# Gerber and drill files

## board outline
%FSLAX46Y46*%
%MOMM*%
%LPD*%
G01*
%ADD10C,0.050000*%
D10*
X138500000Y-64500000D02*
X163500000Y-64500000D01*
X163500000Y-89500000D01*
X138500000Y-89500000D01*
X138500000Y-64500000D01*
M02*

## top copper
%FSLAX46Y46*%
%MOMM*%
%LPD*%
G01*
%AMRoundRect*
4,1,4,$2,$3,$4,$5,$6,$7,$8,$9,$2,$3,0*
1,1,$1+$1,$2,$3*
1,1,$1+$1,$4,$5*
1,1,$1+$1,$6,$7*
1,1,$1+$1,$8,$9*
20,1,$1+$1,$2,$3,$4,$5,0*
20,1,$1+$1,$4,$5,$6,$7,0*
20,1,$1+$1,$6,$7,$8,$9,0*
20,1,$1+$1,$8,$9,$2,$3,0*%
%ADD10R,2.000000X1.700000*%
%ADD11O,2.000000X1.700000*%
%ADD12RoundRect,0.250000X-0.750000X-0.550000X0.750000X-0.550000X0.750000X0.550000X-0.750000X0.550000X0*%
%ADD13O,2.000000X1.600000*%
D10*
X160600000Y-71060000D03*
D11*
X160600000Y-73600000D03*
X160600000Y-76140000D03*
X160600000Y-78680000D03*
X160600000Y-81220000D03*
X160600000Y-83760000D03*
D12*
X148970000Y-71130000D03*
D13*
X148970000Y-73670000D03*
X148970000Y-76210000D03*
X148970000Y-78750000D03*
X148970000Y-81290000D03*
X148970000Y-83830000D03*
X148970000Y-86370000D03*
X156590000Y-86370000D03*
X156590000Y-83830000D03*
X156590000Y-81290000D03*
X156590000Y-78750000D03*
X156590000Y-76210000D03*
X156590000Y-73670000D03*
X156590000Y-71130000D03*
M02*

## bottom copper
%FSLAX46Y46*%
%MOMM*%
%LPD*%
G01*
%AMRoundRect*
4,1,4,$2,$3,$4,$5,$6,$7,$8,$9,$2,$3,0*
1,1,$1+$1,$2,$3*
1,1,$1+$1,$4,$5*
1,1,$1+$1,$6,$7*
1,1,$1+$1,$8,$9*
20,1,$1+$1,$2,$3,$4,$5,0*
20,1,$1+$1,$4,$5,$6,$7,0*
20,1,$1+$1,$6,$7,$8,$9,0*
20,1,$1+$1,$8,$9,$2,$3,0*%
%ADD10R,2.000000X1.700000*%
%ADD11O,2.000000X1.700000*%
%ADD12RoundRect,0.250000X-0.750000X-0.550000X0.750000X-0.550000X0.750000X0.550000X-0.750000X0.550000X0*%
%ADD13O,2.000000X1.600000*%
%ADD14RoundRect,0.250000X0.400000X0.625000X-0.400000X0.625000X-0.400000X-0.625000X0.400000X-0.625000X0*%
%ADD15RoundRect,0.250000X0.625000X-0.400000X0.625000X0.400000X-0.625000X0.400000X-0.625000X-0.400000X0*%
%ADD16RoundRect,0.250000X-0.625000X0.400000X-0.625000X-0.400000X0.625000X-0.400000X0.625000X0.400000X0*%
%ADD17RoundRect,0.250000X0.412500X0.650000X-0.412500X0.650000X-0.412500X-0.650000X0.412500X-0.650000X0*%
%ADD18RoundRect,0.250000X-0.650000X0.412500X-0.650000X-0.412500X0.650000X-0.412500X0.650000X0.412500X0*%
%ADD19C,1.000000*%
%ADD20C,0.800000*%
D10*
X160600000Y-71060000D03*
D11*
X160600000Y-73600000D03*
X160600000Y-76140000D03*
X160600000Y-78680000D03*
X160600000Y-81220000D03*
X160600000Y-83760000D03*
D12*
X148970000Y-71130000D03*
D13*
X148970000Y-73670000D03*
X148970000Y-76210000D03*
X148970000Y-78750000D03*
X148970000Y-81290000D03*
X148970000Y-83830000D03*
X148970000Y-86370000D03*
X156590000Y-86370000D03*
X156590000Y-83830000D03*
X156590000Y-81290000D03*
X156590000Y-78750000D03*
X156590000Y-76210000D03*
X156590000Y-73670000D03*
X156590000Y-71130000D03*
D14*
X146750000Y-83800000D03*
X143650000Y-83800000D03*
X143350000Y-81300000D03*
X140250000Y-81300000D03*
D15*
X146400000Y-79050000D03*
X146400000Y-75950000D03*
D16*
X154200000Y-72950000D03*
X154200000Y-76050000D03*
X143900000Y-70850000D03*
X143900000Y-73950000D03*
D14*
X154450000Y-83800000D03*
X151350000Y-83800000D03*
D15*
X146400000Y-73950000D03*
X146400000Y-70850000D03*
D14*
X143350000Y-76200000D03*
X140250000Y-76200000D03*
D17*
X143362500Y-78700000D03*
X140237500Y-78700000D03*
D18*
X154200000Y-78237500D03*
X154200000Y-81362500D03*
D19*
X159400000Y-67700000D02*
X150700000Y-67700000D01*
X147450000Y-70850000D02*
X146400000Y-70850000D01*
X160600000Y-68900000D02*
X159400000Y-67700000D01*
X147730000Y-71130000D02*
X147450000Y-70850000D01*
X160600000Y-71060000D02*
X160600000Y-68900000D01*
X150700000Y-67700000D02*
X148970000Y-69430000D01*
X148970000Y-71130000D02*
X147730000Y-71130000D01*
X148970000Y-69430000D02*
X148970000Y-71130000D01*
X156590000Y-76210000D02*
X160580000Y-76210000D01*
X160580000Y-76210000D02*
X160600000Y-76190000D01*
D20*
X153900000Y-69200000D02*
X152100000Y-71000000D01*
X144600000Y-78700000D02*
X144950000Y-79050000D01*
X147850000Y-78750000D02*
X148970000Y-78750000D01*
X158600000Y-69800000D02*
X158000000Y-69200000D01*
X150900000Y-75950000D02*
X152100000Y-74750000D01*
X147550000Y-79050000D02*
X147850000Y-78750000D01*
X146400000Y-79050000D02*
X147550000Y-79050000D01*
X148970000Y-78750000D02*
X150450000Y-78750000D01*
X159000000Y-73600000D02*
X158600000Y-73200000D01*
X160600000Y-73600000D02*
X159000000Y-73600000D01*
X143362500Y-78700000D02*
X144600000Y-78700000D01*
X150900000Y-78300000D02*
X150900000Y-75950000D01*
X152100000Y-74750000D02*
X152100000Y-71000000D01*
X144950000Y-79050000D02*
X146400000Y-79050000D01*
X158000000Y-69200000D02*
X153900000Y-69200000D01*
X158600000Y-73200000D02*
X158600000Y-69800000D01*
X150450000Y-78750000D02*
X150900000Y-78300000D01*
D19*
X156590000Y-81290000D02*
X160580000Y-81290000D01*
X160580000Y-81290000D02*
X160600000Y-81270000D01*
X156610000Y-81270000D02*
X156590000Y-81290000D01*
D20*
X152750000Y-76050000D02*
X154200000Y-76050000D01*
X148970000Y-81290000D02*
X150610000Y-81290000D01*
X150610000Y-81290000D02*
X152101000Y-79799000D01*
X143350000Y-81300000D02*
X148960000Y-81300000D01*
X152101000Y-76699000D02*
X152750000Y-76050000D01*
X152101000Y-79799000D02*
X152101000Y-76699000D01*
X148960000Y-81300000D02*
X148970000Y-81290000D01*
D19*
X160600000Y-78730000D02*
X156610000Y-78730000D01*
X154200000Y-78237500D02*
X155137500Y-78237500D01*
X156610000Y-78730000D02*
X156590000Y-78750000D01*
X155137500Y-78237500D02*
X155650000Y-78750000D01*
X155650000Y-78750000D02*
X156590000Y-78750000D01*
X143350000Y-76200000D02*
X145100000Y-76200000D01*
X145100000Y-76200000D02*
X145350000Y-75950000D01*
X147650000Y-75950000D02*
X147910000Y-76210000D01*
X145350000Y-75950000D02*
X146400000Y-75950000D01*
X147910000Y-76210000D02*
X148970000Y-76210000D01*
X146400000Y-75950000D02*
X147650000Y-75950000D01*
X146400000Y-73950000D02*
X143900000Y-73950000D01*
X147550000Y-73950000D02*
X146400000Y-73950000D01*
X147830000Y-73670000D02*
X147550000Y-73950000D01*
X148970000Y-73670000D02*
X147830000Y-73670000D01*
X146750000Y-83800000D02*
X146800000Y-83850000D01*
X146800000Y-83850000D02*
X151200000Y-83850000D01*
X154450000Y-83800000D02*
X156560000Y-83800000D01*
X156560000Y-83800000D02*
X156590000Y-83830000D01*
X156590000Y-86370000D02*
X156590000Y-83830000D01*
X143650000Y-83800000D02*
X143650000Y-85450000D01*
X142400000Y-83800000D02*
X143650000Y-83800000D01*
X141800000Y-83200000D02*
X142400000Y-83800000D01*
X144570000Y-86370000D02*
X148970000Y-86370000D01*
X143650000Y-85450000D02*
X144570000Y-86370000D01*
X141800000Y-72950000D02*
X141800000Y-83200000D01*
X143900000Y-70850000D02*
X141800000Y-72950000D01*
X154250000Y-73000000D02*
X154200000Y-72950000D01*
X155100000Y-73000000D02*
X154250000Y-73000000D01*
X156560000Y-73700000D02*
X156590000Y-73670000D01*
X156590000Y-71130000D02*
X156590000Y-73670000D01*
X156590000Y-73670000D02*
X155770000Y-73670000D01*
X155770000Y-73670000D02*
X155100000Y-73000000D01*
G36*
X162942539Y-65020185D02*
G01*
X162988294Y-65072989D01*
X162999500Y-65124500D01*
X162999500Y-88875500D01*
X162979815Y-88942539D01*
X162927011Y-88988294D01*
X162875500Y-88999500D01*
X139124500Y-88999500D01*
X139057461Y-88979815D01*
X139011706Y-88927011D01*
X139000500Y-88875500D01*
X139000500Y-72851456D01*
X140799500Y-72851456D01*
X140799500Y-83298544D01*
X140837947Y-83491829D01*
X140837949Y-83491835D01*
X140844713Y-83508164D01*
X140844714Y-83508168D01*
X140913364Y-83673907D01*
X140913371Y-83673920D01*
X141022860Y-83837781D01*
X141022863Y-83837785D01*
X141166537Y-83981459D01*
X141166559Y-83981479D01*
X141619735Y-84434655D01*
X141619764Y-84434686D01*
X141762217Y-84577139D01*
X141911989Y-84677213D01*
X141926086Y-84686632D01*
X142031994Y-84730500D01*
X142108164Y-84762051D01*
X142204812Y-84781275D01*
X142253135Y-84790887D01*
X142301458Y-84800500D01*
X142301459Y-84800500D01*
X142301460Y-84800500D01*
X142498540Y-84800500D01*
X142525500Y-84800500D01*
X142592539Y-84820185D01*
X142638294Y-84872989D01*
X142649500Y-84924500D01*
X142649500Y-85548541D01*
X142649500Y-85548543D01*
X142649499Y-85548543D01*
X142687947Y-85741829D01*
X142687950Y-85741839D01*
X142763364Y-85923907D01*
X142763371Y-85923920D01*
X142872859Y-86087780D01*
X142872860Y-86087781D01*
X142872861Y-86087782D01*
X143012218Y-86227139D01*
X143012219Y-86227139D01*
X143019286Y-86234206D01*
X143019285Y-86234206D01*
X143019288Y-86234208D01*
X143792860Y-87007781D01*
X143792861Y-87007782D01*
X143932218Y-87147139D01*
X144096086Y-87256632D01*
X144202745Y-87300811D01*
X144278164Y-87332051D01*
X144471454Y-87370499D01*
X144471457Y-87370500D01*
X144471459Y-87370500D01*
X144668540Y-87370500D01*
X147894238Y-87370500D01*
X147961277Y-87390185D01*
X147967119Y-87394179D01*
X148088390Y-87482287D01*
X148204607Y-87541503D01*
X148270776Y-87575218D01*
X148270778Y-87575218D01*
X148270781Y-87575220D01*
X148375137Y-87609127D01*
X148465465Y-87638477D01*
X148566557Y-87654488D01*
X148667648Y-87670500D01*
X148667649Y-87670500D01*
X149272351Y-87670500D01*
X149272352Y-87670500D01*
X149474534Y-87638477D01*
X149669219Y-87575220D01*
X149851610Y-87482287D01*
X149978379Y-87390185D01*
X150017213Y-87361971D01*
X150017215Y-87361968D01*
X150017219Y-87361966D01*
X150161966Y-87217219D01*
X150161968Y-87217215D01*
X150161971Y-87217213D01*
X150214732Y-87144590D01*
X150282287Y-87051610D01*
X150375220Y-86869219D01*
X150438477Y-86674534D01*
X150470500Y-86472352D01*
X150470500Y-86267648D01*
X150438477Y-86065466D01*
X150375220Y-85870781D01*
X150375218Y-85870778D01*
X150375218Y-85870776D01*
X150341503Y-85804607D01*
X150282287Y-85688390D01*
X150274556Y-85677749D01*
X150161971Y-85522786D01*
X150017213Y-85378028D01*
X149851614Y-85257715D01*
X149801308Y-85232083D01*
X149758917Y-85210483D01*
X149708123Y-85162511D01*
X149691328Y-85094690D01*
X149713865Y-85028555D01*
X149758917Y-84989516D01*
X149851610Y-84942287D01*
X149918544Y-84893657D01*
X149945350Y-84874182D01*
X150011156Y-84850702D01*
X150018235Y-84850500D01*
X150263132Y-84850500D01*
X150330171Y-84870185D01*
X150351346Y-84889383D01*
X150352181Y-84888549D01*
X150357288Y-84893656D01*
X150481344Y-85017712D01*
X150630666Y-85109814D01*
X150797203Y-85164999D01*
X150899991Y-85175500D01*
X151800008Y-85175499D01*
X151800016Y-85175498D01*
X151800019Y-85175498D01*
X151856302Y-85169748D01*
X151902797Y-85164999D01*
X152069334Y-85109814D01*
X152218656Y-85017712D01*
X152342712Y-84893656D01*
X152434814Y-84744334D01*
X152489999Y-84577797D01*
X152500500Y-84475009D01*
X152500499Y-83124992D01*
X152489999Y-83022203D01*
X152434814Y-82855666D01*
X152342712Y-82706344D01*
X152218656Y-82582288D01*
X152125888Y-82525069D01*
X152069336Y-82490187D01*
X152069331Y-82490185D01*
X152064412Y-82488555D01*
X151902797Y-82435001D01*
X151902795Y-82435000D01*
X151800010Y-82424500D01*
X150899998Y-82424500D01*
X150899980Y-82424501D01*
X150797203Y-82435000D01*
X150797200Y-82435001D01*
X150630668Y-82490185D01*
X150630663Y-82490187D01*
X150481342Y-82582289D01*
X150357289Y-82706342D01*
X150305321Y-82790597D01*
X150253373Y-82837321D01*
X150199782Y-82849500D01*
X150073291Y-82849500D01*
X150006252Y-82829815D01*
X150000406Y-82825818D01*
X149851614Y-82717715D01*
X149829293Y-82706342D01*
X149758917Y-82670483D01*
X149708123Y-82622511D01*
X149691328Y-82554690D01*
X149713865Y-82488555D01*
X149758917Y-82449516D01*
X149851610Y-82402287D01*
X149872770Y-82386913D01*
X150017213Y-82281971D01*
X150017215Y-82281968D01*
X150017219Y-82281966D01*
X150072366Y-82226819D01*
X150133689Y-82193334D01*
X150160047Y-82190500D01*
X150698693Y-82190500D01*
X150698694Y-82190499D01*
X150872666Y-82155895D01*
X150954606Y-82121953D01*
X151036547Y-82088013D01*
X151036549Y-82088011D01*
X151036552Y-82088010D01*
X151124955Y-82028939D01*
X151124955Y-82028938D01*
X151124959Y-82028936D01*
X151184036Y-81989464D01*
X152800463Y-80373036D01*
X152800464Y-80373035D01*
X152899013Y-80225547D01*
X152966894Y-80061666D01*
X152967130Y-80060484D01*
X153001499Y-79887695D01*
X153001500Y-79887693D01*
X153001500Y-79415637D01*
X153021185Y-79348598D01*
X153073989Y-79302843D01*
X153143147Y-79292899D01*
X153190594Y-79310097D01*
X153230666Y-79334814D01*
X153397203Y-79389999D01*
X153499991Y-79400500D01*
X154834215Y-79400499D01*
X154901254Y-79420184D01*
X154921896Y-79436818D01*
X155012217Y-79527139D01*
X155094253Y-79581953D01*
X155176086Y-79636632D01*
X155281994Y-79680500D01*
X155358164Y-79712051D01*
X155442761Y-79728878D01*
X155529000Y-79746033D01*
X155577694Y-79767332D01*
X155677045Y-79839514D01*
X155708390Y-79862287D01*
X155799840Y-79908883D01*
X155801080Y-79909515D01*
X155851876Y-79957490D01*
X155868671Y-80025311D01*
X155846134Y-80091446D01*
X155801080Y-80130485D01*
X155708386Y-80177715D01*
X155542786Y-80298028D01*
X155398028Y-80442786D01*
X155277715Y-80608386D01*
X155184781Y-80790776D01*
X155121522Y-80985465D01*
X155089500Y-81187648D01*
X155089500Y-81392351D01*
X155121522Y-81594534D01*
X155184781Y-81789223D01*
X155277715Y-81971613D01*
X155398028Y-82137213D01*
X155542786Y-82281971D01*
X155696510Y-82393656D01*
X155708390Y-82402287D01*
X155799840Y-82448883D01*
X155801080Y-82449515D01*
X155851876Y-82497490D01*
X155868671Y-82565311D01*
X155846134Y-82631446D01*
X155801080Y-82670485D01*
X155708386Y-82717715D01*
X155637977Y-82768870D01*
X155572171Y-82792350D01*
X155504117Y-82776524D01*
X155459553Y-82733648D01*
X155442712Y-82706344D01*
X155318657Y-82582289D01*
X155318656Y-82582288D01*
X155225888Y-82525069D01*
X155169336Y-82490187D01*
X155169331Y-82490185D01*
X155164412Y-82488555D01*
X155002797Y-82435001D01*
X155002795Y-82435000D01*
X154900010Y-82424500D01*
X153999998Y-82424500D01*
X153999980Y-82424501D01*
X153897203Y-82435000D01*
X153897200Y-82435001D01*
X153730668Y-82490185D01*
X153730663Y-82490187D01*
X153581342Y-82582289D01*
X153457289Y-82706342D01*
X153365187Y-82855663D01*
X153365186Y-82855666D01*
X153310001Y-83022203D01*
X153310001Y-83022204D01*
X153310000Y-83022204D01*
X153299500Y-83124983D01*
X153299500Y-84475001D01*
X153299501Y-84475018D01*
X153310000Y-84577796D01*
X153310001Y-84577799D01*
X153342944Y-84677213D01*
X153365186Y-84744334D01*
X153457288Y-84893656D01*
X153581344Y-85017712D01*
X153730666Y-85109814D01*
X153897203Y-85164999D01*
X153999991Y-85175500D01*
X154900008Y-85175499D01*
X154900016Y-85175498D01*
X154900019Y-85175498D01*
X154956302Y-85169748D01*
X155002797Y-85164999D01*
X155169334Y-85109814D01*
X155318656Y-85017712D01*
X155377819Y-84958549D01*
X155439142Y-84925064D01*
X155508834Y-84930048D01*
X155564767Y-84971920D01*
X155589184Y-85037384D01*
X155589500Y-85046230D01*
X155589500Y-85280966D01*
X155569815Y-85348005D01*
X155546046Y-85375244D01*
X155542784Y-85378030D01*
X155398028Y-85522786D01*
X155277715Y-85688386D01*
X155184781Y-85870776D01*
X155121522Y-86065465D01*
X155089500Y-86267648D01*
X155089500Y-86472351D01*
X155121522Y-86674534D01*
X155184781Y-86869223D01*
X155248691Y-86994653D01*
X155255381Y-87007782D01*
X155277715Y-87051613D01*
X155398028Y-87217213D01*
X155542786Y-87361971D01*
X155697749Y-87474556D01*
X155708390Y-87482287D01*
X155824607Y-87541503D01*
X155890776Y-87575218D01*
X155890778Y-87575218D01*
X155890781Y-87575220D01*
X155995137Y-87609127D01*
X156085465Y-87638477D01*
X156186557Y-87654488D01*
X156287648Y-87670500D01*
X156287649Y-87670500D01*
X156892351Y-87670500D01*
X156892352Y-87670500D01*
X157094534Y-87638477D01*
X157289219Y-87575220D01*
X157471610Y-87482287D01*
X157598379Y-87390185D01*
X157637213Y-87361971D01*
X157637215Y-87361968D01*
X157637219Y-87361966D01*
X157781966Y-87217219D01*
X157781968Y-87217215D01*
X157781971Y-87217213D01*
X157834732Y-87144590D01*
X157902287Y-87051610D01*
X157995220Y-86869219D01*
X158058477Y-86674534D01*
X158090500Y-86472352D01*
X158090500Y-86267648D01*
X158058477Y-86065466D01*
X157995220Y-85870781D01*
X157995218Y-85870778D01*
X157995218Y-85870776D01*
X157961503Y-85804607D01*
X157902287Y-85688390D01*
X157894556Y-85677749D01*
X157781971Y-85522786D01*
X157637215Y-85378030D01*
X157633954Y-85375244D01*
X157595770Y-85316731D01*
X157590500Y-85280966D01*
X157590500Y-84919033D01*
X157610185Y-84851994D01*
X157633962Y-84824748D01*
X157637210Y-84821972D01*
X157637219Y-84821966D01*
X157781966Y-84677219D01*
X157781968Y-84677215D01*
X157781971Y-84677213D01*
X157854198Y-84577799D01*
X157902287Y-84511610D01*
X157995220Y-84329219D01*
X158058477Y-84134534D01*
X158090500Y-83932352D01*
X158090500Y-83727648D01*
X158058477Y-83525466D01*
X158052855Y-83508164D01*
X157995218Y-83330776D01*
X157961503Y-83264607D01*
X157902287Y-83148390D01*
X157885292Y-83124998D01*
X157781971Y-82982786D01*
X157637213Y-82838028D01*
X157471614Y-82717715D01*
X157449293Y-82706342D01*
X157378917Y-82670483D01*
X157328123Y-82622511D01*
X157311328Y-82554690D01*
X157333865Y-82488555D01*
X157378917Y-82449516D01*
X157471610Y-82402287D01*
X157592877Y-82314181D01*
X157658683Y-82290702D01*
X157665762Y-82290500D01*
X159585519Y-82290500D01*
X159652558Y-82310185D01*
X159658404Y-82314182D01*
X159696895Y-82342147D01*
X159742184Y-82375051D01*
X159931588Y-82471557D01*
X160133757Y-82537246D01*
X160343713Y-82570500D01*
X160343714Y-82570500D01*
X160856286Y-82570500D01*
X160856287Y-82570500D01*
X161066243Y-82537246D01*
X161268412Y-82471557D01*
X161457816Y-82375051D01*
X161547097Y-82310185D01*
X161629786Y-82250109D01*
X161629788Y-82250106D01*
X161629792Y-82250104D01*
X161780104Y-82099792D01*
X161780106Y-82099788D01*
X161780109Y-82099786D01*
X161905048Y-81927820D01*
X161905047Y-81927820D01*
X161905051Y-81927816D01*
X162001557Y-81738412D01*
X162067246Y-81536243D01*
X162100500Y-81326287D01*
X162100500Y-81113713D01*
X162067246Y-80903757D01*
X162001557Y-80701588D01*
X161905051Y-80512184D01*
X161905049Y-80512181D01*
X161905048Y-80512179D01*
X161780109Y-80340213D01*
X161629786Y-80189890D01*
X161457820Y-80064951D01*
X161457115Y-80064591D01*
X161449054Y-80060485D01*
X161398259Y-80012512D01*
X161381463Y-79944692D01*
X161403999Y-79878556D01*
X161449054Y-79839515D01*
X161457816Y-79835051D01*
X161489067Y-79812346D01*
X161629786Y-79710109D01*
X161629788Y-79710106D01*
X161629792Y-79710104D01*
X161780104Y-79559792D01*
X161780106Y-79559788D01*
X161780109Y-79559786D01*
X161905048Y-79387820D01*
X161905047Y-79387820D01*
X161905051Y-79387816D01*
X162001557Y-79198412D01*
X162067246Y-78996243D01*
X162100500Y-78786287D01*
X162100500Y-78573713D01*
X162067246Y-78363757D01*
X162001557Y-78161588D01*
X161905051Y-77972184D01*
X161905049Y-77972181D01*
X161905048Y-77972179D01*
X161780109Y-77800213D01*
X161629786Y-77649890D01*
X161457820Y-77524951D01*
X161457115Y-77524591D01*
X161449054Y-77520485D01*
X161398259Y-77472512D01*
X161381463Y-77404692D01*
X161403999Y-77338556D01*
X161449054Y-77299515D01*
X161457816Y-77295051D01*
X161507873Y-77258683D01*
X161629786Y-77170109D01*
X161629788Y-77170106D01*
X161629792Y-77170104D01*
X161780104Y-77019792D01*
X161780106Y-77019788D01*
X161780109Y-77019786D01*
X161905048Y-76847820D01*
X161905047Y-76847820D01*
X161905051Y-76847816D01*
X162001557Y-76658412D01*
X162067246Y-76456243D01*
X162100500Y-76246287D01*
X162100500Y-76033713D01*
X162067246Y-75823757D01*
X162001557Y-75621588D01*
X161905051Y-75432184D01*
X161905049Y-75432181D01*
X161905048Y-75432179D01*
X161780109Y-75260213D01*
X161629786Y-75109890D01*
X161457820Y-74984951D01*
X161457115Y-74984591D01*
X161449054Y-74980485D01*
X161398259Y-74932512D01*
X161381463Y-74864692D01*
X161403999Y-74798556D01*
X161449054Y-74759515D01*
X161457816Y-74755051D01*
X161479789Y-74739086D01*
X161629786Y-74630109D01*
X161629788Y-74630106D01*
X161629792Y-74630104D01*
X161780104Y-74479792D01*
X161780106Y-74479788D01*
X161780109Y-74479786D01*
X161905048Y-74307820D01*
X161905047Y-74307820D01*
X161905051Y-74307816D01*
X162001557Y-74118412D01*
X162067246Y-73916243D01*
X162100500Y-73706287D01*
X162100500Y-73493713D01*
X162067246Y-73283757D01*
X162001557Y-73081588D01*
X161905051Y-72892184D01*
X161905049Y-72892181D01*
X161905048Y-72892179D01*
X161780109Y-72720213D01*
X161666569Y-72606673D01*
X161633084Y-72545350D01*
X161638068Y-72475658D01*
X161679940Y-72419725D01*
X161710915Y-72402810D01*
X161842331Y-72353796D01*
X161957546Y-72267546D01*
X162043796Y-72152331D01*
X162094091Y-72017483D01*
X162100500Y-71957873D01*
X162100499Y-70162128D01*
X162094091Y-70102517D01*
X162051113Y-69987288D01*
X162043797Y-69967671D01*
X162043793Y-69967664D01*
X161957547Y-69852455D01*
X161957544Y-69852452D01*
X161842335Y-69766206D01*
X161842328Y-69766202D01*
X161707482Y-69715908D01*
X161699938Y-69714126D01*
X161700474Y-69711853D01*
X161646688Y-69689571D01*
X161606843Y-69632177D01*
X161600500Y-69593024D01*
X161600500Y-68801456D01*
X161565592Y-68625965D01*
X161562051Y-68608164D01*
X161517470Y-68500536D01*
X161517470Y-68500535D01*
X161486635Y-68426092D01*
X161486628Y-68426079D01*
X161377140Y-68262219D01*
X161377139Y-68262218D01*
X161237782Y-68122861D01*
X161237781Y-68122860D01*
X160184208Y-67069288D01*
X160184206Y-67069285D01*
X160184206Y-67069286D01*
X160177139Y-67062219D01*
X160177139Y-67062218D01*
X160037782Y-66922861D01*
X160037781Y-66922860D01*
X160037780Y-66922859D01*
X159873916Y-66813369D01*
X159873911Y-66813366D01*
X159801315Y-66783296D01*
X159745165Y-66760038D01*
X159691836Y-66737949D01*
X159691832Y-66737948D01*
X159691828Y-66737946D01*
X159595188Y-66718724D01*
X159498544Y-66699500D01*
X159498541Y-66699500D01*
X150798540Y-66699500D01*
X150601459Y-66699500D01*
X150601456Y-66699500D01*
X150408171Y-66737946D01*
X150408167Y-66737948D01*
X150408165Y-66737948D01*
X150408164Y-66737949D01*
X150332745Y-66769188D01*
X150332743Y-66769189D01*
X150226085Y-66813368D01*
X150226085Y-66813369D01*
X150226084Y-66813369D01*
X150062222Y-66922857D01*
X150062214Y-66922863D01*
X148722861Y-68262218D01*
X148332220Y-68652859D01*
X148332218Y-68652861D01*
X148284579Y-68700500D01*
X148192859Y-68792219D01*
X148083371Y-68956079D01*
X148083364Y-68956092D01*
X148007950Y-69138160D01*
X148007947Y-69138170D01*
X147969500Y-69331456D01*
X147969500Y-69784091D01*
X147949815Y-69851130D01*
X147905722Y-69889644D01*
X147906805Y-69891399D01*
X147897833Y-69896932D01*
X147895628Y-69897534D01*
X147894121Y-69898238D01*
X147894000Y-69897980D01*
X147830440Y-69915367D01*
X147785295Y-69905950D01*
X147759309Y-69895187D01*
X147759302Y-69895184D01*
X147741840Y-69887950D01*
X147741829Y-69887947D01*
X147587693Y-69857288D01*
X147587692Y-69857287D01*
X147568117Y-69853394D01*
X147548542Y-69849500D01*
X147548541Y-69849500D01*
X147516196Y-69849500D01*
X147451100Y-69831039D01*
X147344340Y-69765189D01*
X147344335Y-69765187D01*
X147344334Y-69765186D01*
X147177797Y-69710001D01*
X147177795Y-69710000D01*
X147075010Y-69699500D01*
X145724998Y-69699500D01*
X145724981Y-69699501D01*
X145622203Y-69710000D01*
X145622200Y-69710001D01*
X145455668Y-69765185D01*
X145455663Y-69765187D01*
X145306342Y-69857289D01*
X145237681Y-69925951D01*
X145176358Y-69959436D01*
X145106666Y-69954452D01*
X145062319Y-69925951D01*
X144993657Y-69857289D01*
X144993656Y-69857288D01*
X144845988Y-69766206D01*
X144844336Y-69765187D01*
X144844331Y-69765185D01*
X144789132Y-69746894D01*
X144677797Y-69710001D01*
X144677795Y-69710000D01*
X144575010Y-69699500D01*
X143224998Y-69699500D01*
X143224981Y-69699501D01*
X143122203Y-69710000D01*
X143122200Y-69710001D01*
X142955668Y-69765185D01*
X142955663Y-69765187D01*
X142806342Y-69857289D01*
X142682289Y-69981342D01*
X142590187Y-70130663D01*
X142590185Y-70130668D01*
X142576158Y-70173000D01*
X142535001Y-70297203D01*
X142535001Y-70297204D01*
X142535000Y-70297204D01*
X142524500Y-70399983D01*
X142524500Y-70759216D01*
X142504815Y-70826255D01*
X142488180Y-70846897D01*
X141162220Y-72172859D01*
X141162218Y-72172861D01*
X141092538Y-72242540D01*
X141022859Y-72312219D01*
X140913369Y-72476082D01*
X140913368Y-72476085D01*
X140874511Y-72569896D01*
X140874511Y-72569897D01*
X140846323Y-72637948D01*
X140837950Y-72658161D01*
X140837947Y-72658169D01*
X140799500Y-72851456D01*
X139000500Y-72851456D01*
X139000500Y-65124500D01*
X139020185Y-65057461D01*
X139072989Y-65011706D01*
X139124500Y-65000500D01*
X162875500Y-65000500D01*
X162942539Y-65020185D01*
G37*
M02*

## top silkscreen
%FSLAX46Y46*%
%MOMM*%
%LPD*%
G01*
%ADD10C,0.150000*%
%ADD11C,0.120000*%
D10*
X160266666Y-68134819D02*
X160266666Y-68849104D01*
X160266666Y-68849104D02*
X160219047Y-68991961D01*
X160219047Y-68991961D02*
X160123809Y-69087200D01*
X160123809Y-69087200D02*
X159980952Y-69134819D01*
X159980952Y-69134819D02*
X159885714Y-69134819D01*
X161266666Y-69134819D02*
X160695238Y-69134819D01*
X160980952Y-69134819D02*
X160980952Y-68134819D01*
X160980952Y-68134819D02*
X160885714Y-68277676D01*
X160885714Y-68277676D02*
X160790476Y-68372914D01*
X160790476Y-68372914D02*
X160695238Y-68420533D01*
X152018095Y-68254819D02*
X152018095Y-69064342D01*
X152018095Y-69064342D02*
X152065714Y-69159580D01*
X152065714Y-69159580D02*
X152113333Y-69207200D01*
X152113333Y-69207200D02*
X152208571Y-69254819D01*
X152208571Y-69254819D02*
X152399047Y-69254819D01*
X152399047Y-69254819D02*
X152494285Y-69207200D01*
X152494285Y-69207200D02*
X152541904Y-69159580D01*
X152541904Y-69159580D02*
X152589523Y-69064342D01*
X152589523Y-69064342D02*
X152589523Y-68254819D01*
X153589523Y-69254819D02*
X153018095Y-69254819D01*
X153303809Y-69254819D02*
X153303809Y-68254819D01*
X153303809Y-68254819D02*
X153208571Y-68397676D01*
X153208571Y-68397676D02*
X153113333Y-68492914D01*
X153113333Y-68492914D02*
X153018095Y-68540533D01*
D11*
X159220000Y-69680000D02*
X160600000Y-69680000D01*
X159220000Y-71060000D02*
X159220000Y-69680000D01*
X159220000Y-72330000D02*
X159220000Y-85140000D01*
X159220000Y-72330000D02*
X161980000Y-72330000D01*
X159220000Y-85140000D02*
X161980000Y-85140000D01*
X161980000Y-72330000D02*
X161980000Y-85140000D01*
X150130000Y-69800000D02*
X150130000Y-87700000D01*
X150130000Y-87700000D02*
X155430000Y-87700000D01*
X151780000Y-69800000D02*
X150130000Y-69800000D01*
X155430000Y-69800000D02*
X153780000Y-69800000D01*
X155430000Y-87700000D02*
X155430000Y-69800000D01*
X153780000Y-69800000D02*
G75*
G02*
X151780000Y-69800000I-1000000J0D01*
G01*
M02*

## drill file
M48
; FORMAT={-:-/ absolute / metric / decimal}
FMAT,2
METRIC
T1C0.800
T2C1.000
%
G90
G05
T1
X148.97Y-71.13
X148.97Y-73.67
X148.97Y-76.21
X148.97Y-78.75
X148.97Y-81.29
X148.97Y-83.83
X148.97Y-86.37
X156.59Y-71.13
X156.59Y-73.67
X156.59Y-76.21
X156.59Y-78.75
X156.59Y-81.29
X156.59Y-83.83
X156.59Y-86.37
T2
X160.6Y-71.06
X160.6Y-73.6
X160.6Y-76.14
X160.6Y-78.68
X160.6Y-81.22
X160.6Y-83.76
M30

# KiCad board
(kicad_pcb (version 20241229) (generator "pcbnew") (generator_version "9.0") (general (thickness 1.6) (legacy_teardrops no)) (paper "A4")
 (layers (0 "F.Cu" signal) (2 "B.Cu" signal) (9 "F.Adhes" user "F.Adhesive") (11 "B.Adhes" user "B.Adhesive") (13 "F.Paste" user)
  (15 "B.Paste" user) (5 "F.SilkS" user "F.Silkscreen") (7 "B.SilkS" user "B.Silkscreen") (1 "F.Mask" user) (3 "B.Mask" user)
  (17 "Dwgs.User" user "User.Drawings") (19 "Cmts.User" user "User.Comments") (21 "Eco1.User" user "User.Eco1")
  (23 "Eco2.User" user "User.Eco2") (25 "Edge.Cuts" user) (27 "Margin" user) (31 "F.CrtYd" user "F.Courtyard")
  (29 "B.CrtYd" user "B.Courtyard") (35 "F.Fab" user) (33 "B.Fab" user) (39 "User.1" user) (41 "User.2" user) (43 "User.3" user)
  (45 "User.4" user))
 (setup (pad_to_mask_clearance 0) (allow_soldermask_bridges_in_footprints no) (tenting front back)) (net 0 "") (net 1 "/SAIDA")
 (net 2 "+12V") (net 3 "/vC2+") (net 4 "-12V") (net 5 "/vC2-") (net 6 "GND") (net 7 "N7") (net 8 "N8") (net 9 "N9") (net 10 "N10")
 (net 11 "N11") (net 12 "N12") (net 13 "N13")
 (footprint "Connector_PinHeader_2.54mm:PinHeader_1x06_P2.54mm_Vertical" (layer "F.Cu") (at 160.6 71.06)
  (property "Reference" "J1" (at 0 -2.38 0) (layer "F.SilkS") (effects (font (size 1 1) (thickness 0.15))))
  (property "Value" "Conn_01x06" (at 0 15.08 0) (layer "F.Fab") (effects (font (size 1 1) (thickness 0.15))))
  (fp_line (start -1.38 -1.38) (end 0 -1.38) (stroke (width 0.12) (type solid)) (layer "F.SilkS"))
  (fp_line (start -1.38 0) (end -1.38 -1.38) (stroke (width 0.12) (type solid)) (layer "F.SilkS"))
  (fp_line (start -1.38 1.27) (end -1.38 14.08) (stroke (width 0.12) (type solid)) (layer "F.SilkS"))
  (fp_line (start -1.38 1.27) (end 1.38 1.27) (stroke (width 0.12) (type solid)) (layer "F.SilkS"))
  (fp_line (start -1.38 14.08) (end 1.38 14.08) (stroke (width 0.12) (type solid)) (layer "F.SilkS"))
  (fp_line (start 1.38 1.27) (end 1.38 14.08) (stroke (width 0.12) (type solid)) (layer "F.SilkS"))
  (pad "1" thru_hole rect (at 0 0) (size 2 1.7) (drill 1) (layers "*.Cu" "*.Mask") (remove_unused_layers no) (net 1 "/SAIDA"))
  (pad "2" thru_hole oval (at 0 2.54) (size 2 1.7) (drill 1) (layers "*.Cu" "*.Mask") (remove_unused_layers no) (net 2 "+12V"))
  (pad "3" thru_hole oval (at 0 5.08) (size 2 1.7) (drill 1) (layers "*.Cu" "*.Mask") (remove_unused_layers no) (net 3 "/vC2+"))
  (pad "4" thru_hole oval (at 0 7.62) (size 2 1.7) (drill 1) (layers "*.Cu" "*.Mask") (remove_unused_layers no) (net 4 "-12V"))
  (pad "5" thru_hole oval (at 0 10.16) (size 2 1.7) (drill 1) (layers "*.Cu" "*.Mask") (remove_unused_layers no) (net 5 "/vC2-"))
  (pad "6" thru_hole oval (at 0 12.7) (size 2 1.7) (drill 1) (layers "*.Cu" "*.Mask") (remove_unused_layers no) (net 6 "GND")))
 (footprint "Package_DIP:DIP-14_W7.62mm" (layer "F.Cu") (at 148.97 71.13)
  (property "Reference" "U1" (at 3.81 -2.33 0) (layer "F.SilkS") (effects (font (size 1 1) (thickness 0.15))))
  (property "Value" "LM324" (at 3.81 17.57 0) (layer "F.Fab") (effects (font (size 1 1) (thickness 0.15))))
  (fp_line (start 1.16 -1.33) (end 1.16 16.57) (stroke (width 0.12) (type solid)) (layer "F.SilkS"))
  (fp_line (start 1.16 16.57) (end 6.46 16.57) (stroke (width 0.12) (type solid)) (layer "F.SilkS"))
  (fp_line (start 2.81 -1.33) (end 1.16 -1.33) (stroke (width 0.12) (type solid)) (layer "F.SilkS"))
  (fp_line (start 6.46 -1.33) (end 4.81 -1.33) (stroke (width 0.12) (type solid)) (layer "F.SilkS"))
  (fp_line (start 6.46 16.57) (end 6.46 -1.33) (stroke (width 0.12) (type solid)) (layer "F.SilkS"))
  (fp_arc (start 4.81 -1.33) (mid 3.81 -0.33) (end 2.81 -1.33) (stroke (width 0.12) (type solid)) (layer "F.SilkS"))
  (pad "1" thru_hole roundrect (at 0 0) (size 2 1.6) (drill 0.8) (layers "*.Cu" "*.Mask") (remove_unused_layers no)
   (roundrect_rratio 0.15625) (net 1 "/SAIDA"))
  (pad "2" thru_hole oval (at 0 2.54) (size 2 1.6) (drill 0.8) (layers "*.Cu" "*.Mask") (remove_unused_layers no) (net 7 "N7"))
  (pad "3" thru_hole oval (at 0 5.08) (size 2 1.6) (drill 0.8) (layers "*.Cu" "*.Mask") (remove_unused_layers no) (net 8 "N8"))
  (pad "4" thru_hole oval (at 0 7.62) (size 2 1.6) (drill 0.8) (layers "*.Cu" "*.Mask") (remove_unused_layers no) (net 2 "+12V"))
  (pad "5" thru_hole oval (at 0 10.16) (size 2 1.6) (drill 0.8) (layers "*.Cu" "*.Mask") (remove_unused_layers no) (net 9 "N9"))
  (pad "6" thru_hole oval (at 0 12.7) (size 2 1.6) (drill 0.8) (layers "*.Cu" "*.Mask") (remove_unused_layers no) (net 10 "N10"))
  (pad "7" thru_hole oval (at 0 15.24) (size 2 1.6) (drill 0.8) (layers "*.Cu" "*.Mask") (remove_unused_layers no) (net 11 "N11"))
  (pad "8" thru_hole oval (at 7.62 15.24) (size 2 1.6) (drill 0.8) (layers "*.Cu" "*.Mask") (remove_unused_layers no) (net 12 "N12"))
  (pad "9" thru_hole oval (at 7.62 12.7) (size 2 1.6) (drill 0.8) (layers "*.Cu" "*.Mask") (remove_unused_layers no) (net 12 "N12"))
  (pad "10" thru_hole oval (at 7.62 10.16) (size 2 1.6) (drill 0.8) (layers "*.Cu" "*.Mask") (remove_unused_layers no) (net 5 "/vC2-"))
  (pad "11" thru_hole oval (at 7.62 7.62) (size 2 1.6) (drill 0.8) (layers "*.Cu" "*.Mask") (remove_unused_layers no) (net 4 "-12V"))
  (pad "12" thru_hole oval (at 7.62 5.08) (size 2 1.6) (drill 0.8) (layers "*.Cu" "*.Mask") (remove_unused_layers no) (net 3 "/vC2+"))
  (pad "13" thru_hole oval (at 7.62 2.54) (size 2 1.6) (drill 0.8) (layers "*.Cu" "*.Mask") (remove_unused_layers no) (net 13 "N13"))
  (pad "14" thru_hole oval (at 7.62 0) (size 2 1.6) (drill 0.8) (layers "*.Cu" "*.Mask") (remove_unused_layers no) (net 13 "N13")))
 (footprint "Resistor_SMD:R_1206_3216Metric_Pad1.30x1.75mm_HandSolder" (layer "B.Cu") (at 145.2 83.8 180)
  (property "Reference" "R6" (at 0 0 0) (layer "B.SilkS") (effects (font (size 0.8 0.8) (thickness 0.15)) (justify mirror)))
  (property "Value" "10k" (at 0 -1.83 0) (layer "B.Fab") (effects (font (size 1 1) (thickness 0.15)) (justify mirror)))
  (pad "1" smd roundrect (at -1.55 0 180) (size 1.3 1.75) (layers "B.Cu" "B.Mask" "B.Paste") (roundrect_rratio 0.192308) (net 10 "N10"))
  (pad "2" smd roundrect (at 1.55 0 180) (size 1.3 1.75) (layers "B.Cu" "B.Mask" "B.Paste") (roundrect_rratio 0.192308) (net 11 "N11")))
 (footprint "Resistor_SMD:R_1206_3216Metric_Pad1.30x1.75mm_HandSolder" (layer "B.Cu") (at 141.8 81.3 180)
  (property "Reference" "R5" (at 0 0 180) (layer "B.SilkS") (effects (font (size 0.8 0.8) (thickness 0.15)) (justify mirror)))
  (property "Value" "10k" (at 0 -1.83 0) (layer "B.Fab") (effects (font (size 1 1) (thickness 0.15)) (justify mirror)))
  (pad "1" smd roundrect (at -1.55 0 180) (size 1.3 1.75) (layers "B.Cu" "B.Mask" "B.Paste") (roundrect_rratio 0.192308) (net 9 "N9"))
  (pad "2" smd roundrect (at 1.55 0 180) (size 1.3 1.75) (layers "B.Cu" "B.Mask" "B.Paste") (roundrect_rratio 0.192308) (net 6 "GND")))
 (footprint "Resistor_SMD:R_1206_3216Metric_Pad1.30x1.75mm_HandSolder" (layer "B.Cu") (at 146.4 77.5 90)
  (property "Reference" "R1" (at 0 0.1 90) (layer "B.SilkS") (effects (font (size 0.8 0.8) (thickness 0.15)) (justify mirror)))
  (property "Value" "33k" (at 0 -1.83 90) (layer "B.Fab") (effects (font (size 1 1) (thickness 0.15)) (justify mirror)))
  (pad "1" smd roundrect (at -1.55 0 90) (size 1.3 1.75) (layers "B.Cu" "B.Mask" "B.Paste") (roundrect_rratio 0.192308) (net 2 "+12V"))
  (pad "2" smd roundrect (at 1.55 0 90) (size 1.3 1.75) (layers "B.Cu" "B.Mask" "B.Paste") (roundrect_rratio 0.192308) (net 8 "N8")))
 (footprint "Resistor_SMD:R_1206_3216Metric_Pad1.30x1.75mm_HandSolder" (layer "B.Cu") (at 154.2 74.5 -90)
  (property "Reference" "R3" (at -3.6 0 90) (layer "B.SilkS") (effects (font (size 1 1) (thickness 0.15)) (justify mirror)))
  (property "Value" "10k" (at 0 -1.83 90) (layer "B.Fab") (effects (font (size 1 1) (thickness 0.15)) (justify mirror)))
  (pad "1" smd roundrect (at -1.55 0 270) (size 1.3 1.75) (layers "B.Cu" "B.Mask" "B.Paste") (roundrect_rratio 0.192308) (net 13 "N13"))
  (pad "2" smd roundrect (at 1.55 0 270) (size 1.3 1.75) (layers "B.Cu" "B.Mask" "B.Paste") (roundrect_rratio 0.192308) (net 9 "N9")))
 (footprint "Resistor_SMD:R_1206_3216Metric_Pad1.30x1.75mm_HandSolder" (layer "B.Cu") (at 143.9 72.4 -90)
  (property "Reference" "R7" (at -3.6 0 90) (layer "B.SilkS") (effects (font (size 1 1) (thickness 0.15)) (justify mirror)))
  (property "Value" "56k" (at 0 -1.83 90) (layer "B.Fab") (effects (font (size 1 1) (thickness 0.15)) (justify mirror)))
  (pad "1" smd roundrect (at -1.55 0 270) (size 1.3 1.75) (layers "B.Cu" "B.Mask" "B.Paste") (roundrect_rratio 0.192308) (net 11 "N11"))
  (pad "2" smd roundrect (at 1.55 0 270) (size 1.3 1.75) (layers "B.Cu" "B.Mask" "B.Paste") (roundrect_rratio 0.192308) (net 7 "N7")))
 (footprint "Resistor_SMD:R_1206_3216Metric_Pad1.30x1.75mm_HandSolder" (layer "B.Cu") (at 152.9 83.8 180)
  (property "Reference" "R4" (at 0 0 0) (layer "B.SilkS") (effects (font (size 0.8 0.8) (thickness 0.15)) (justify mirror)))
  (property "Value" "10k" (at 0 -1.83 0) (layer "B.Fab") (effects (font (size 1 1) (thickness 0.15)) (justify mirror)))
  (pad "1" smd roundrect (at -1.55 0 180) (size 1.3 1.75) (layers "B.Cu" "B.Mask" "B.Paste") (roundrect_rratio 0.192308) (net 12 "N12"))
  (pad "2" smd roundrect (at 1.55 0 180) (size 1.3 1.75) (layers "B.Cu" "B.Mask" "B.Paste") (roundrect_rratio 0.192308) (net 10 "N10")))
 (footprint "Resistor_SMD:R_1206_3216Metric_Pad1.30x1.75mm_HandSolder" (layer "B.Cu") (at 146.4 72.4 90)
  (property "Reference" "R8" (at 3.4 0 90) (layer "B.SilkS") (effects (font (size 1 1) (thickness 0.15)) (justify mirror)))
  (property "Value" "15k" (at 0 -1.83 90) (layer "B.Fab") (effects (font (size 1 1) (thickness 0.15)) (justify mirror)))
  (pad "1" smd roundrect (at -1.55 0 90) (size 1.3 1.75) (layers "B.Cu" "B.Mask" "B.Paste") (roundrect_rratio 0.192308) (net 7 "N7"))
  (pad "2" smd roundrect (at 1.55 0 90) (size 1.3 1.75) (layers "B.Cu" "B.Mask" "B.Paste") (roundrect_rratio 0.192308) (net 1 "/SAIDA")))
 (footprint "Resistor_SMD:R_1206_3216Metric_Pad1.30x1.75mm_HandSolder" (layer "B.Cu") (at 141.8 76.2 180)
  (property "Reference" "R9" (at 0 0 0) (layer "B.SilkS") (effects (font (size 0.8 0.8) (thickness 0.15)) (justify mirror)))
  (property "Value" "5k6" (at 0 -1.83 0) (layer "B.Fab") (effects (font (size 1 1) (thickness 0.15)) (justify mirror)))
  (pad "1" smd roundrect (at -1.55 0 180) (size 1.3 1.75) (layers "B.Cu" "B.Mask" "B.Paste") (roundrect_rratio 0.192308) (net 8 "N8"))
  (pad "2" smd roundrect (at 1.55 0 180) (size 1.3 1.75) (layers "B.Cu" "B.Mask" "B.Paste") (roundrect_rratio 0.192308) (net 6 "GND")))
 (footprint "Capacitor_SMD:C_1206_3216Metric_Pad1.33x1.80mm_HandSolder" (layer "B.Cu") (at 141.8 78.7 180)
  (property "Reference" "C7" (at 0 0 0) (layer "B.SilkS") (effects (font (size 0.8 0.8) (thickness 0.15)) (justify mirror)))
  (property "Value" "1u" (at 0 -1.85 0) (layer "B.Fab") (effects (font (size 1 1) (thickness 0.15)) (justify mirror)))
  (pad "1" smd roundrect (at -1.5625 0 180) (size 1.325 1.8) (layers "B.Cu" "B.Mask" "B.Paste") (roundrect_rratio 0.188679) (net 2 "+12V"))
  (pad "2" smd roundrect (at 1.5625 0 180) (size 1.325 1.8) (layers "B.Cu" "B.Mask" "B.Paste") (roundrect_rratio 0.188679) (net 6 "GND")))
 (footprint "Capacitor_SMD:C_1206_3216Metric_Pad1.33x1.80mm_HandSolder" (layer "B.Cu") (at 154.2 79.8 -90)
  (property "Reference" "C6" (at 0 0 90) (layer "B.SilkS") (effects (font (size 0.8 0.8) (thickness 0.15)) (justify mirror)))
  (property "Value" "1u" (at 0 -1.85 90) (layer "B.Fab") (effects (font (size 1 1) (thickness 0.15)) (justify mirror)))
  (pad "1" smd roundrect (at -1.5625 0 270) (size 1.325 1.8) (layers "B.Cu" "B.Mask" "B.Paste") (roundrect_rratio 0.188679) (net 4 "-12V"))
  (pad "2" smd roundrect (at 1.5625 0 270) (size 1.325 1.8) (layers "B.Cu" "B.Mask" "B.Paste") (roundrect_rratio 0.188679) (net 6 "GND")))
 (gr_rect (start 138.5 64.5) (end 163.5 89.5) (stroke (width 0.05) (type default)) (fill no) (layer "Edge.Cuts"))
 (segment (start 159.4 67.7) (end 150.7 67.7) (width 1) (layer "B.Cu") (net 1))
 (segment (start 147.45 70.85) (end 146.4 70.85) (width 1) (layer "B.Cu") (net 1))
 (segment (start 160.6 68.9) (end 159.4 67.7) (width 1) (layer "B.Cu") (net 1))
 (segment (start 147.73 71.13) (end 147.45 70.85) (width 1) (layer "B.Cu") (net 1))
 (segment (start 160.6 71.06) (end 160.6 68.9) (width 1) (layer "B.Cu") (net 1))
 (segment (start 150.7 67.7) (end 148.97 69.43) (width 1) (layer "B.Cu") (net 1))
 (segment (start 148.97 71.13) (end 147.73 71.13) (width 1) (layer "B.Cu") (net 1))
 (segment (start 148.97 69.43) (end 148.97 71.13) (width 1) (layer "B.Cu") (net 1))
 (segment (start 156.59 76.21) (end 160.58 76.21) (width 1) (layer "B.Cu") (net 3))
 (segment (start 160.58 76.21) (end 160.6 76.19) (width 1) (layer "B.Cu") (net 3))
 (segment (start 153.9 69.2) (end 152.1 71) (width 0.8) (layer "B.Cu") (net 2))
 (segment (start 144.6 78.7) (end 144.95 79.05) (width 0.8) (layer "B.Cu") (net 2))
 (segment (start 147.85 78.75) (end 148.97 78.75) (width 0.8) (layer "B.Cu") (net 2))
 (segment (start 158.6 69.8) (end 158 69.2) (width 0.8) (layer "B.Cu") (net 2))
 (segment (start 150.9 75.95) (end 152.1 74.75) (width 0.8) (layer "B.Cu") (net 2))
 (segment (start 147.55 79.05) (end 147.85 78.75) (width 0.8) (layer "B.Cu") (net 2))
 (segment (start 146.4 79.05) (end 147.55 79.05) (width 0.8) (layer "B.Cu") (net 2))
 (segment (start 148.97 78.75) (end 150.45 78.75) (width 0.8) (layer "B.Cu") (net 2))
 (segment (start 159 73.6) (end 158.6 73.2) (width 0.8) (layer "B.Cu") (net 2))
 (segment (start 160.6 73.6) (end 159 73.6) (width 0.8) (layer "B.Cu") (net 2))
 (segment (start 143.3625 78.7) (end 144.6 78.7) (width 0.8) (layer "B.Cu") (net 2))
 (segment (start 150.9 78.3) (end 150.9 75.95) (width 0.8) (layer "B.Cu") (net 2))
 (segment (start 152.1 74.75) (end 152.1 71) (width 0.8) (layer "B.Cu") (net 2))
 (segment (start 144.95 79.05) (end 146.4 79.05) (width 0.8) (layer "B.Cu") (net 2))
 (segment (start 158 69.2) (end 153.9 69.2) (width 0.8) (layer "B.Cu") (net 2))
 (segment (start 158.6 73.2) (end 158.6 69.8) (width 0.8) (layer "B.Cu") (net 2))
 (segment (start 150.45 78.75) (end 150.9 78.3) (width 0.8) (layer "B.Cu") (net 2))
 (segment (start 156.59 81.29) (end 160.58 81.29) (width 1) (layer "B.Cu") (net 5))
 (segment (start 160.58 81.29) (end 160.6 81.27) (width 1) (layer "B.Cu") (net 5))
 (segment (start 156.61 81.27) (end 156.59 81.29) (width 1) (layer "B.Cu") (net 5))
 (segment (start 152.75 76.05) (end 154.2 76.05) (width 0.8) (layer "B.Cu") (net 9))
 (segment (start 148.97 81.29) (end 150.61 81.29) (width 0.8) (layer "B.Cu") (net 9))
 (segment (start 150.61 81.29) (end 152.101 79.799) (width 0.8) (layer "B.Cu") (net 9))
 (segment (start 143.35 81.3) (end 148.96 81.3) (width 0.8) (layer "B.Cu") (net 9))
 (segment (start 152.101 76.699) (end 152.75 76.05) (width 0.8) (layer "B.Cu") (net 9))
 (segment (start 152.101 79.799) (end 152.101 76.699) (width 0.8) (layer "B.Cu") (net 9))
 (segment (start 148.96 81.3) (end 148.97 81.29) (width 0.8) (layer "B.Cu") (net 9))
 (segment (start 160.6 78.73) (end 156.61 78.73) (width 1) (layer "B.Cu") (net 4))
 (segment (start 154.2 78.2375) (end 155.1375 78.2375) (width 1) (layer "B.Cu") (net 4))
 (segment (start 156.61 78.73) (end 156.59 78.75) (width 1) (layer "B.Cu") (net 4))
 (segment (start 155.1375 78.2375) (end 155.65 78.75) (width 1) (layer "B.Cu") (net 4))
 (segment (start 155.65 78.75) (end 156.59 78.75) (width 1) (layer "B.Cu") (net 4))
 (segment (start 143.35 76.2) (end 145.1 76.2) (width 1) (layer "B.Cu") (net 8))
 (segment (start 145.1 76.2) (end 145.35 75.95) (width 1) (layer "B.Cu") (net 8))
 (segment (start 147.65 75.95) (end 147.91 76.21) (width 1) (layer "B.Cu") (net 8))
 (segment (start 145.35 75.95) (end 146.4 75.95) (width 1) (layer "B.Cu") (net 8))
 (segment (start 147.91 76.21) (end 148.97 76.21) (width 1) (layer "B.Cu") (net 8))
 (segment (start 146.4 75.95) (end 147.65 75.95) (width 1) (layer "B.Cu") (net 8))
 (segment (start 146.4 73.95) (end 143.9 73.95) (width 1) (layer "B.Cu") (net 7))
 (segment (start 147.55 73.95) (end 146.4 73.95) (width 1) (layer "B.Cu") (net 7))
 (segment (start 147.83 73.67) (end 147.55 73.95) (width 1) (layer "B.Cu") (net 7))
 (segment (start 148.97 73.67) (end 147.83 73.67) (width 1) (layer "B.Cu") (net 7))
 (segment (start 146.75 83.8) (end 146.8 83.85) (width 1) (layer "B.Cu") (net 10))
 (segment (start 146.8 83.85) (end 151.2 83.85) (width 1) (layer "B.Cu") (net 10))
 (segment (start 154.45 83.8) (end 156.56 83.8) (width 1) (layer "B.Cu") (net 12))
 (segment (start 156.56 83.8) (end 156.59 83.83) (width 1) (layer "B.Cu") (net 12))
 (segment (start 156.59 86.37) (end 156.59 83.83) (width 1) (layer "B.Cu") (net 12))
 (segment (start 143.65 83.8) (end 143.65 85.45) (width 1) (layer "B.Cu") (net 11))
 (segment (start 142.4 83.8) (end 143.65 83.8) (width 1) (layer "B.Cu") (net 11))
 (segment (start 141.8 83.2) (end 142.4 83.8) (width 1) (layer "B.Cu") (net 11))
 (segment (start 144.57 86.37) (end 148.97 86.37) (width 1) (layer "B.Cu") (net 11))
 (segment (start 143.65 85.45) (end 144.57 86.37) (width 1) (layer "B.Cu") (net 11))
 (segment (start 141.8 72.95) (end 141.8 83.2) (width 1) (layer "B.Cu") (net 11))
 (segment (start 143.9 70.85) (end 141.8 72.95) (width 1) (layer "B.Cu") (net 11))
 (segment (start 154.25 73) (end 154.2 72.95) (width 1) (layer "B.Cu") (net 13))
 (segment (start 155.1 73) (end 154.25 73) (width 1) (layer "B.Cu") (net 13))
 (segment (start 156.56 73.7) (end 156.59 73.67) (width 1) (layer "B.Cu") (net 13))
 (segment (start 156.59 71.13) (end 156.59 73.67) (width 1) (layer "B.Cu") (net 13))
 (segment (start 156.59 73.67) (end 155.77 73.67) (width 1) (layer "B.Cu") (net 13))
 (segment (start 155.77 73.67) (end 155.1 73) (width 1) (layer "B.Cu") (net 13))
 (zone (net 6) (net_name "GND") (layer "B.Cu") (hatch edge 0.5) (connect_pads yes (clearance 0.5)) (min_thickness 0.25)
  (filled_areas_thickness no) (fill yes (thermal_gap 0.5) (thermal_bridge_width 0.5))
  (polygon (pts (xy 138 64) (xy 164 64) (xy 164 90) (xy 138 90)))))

